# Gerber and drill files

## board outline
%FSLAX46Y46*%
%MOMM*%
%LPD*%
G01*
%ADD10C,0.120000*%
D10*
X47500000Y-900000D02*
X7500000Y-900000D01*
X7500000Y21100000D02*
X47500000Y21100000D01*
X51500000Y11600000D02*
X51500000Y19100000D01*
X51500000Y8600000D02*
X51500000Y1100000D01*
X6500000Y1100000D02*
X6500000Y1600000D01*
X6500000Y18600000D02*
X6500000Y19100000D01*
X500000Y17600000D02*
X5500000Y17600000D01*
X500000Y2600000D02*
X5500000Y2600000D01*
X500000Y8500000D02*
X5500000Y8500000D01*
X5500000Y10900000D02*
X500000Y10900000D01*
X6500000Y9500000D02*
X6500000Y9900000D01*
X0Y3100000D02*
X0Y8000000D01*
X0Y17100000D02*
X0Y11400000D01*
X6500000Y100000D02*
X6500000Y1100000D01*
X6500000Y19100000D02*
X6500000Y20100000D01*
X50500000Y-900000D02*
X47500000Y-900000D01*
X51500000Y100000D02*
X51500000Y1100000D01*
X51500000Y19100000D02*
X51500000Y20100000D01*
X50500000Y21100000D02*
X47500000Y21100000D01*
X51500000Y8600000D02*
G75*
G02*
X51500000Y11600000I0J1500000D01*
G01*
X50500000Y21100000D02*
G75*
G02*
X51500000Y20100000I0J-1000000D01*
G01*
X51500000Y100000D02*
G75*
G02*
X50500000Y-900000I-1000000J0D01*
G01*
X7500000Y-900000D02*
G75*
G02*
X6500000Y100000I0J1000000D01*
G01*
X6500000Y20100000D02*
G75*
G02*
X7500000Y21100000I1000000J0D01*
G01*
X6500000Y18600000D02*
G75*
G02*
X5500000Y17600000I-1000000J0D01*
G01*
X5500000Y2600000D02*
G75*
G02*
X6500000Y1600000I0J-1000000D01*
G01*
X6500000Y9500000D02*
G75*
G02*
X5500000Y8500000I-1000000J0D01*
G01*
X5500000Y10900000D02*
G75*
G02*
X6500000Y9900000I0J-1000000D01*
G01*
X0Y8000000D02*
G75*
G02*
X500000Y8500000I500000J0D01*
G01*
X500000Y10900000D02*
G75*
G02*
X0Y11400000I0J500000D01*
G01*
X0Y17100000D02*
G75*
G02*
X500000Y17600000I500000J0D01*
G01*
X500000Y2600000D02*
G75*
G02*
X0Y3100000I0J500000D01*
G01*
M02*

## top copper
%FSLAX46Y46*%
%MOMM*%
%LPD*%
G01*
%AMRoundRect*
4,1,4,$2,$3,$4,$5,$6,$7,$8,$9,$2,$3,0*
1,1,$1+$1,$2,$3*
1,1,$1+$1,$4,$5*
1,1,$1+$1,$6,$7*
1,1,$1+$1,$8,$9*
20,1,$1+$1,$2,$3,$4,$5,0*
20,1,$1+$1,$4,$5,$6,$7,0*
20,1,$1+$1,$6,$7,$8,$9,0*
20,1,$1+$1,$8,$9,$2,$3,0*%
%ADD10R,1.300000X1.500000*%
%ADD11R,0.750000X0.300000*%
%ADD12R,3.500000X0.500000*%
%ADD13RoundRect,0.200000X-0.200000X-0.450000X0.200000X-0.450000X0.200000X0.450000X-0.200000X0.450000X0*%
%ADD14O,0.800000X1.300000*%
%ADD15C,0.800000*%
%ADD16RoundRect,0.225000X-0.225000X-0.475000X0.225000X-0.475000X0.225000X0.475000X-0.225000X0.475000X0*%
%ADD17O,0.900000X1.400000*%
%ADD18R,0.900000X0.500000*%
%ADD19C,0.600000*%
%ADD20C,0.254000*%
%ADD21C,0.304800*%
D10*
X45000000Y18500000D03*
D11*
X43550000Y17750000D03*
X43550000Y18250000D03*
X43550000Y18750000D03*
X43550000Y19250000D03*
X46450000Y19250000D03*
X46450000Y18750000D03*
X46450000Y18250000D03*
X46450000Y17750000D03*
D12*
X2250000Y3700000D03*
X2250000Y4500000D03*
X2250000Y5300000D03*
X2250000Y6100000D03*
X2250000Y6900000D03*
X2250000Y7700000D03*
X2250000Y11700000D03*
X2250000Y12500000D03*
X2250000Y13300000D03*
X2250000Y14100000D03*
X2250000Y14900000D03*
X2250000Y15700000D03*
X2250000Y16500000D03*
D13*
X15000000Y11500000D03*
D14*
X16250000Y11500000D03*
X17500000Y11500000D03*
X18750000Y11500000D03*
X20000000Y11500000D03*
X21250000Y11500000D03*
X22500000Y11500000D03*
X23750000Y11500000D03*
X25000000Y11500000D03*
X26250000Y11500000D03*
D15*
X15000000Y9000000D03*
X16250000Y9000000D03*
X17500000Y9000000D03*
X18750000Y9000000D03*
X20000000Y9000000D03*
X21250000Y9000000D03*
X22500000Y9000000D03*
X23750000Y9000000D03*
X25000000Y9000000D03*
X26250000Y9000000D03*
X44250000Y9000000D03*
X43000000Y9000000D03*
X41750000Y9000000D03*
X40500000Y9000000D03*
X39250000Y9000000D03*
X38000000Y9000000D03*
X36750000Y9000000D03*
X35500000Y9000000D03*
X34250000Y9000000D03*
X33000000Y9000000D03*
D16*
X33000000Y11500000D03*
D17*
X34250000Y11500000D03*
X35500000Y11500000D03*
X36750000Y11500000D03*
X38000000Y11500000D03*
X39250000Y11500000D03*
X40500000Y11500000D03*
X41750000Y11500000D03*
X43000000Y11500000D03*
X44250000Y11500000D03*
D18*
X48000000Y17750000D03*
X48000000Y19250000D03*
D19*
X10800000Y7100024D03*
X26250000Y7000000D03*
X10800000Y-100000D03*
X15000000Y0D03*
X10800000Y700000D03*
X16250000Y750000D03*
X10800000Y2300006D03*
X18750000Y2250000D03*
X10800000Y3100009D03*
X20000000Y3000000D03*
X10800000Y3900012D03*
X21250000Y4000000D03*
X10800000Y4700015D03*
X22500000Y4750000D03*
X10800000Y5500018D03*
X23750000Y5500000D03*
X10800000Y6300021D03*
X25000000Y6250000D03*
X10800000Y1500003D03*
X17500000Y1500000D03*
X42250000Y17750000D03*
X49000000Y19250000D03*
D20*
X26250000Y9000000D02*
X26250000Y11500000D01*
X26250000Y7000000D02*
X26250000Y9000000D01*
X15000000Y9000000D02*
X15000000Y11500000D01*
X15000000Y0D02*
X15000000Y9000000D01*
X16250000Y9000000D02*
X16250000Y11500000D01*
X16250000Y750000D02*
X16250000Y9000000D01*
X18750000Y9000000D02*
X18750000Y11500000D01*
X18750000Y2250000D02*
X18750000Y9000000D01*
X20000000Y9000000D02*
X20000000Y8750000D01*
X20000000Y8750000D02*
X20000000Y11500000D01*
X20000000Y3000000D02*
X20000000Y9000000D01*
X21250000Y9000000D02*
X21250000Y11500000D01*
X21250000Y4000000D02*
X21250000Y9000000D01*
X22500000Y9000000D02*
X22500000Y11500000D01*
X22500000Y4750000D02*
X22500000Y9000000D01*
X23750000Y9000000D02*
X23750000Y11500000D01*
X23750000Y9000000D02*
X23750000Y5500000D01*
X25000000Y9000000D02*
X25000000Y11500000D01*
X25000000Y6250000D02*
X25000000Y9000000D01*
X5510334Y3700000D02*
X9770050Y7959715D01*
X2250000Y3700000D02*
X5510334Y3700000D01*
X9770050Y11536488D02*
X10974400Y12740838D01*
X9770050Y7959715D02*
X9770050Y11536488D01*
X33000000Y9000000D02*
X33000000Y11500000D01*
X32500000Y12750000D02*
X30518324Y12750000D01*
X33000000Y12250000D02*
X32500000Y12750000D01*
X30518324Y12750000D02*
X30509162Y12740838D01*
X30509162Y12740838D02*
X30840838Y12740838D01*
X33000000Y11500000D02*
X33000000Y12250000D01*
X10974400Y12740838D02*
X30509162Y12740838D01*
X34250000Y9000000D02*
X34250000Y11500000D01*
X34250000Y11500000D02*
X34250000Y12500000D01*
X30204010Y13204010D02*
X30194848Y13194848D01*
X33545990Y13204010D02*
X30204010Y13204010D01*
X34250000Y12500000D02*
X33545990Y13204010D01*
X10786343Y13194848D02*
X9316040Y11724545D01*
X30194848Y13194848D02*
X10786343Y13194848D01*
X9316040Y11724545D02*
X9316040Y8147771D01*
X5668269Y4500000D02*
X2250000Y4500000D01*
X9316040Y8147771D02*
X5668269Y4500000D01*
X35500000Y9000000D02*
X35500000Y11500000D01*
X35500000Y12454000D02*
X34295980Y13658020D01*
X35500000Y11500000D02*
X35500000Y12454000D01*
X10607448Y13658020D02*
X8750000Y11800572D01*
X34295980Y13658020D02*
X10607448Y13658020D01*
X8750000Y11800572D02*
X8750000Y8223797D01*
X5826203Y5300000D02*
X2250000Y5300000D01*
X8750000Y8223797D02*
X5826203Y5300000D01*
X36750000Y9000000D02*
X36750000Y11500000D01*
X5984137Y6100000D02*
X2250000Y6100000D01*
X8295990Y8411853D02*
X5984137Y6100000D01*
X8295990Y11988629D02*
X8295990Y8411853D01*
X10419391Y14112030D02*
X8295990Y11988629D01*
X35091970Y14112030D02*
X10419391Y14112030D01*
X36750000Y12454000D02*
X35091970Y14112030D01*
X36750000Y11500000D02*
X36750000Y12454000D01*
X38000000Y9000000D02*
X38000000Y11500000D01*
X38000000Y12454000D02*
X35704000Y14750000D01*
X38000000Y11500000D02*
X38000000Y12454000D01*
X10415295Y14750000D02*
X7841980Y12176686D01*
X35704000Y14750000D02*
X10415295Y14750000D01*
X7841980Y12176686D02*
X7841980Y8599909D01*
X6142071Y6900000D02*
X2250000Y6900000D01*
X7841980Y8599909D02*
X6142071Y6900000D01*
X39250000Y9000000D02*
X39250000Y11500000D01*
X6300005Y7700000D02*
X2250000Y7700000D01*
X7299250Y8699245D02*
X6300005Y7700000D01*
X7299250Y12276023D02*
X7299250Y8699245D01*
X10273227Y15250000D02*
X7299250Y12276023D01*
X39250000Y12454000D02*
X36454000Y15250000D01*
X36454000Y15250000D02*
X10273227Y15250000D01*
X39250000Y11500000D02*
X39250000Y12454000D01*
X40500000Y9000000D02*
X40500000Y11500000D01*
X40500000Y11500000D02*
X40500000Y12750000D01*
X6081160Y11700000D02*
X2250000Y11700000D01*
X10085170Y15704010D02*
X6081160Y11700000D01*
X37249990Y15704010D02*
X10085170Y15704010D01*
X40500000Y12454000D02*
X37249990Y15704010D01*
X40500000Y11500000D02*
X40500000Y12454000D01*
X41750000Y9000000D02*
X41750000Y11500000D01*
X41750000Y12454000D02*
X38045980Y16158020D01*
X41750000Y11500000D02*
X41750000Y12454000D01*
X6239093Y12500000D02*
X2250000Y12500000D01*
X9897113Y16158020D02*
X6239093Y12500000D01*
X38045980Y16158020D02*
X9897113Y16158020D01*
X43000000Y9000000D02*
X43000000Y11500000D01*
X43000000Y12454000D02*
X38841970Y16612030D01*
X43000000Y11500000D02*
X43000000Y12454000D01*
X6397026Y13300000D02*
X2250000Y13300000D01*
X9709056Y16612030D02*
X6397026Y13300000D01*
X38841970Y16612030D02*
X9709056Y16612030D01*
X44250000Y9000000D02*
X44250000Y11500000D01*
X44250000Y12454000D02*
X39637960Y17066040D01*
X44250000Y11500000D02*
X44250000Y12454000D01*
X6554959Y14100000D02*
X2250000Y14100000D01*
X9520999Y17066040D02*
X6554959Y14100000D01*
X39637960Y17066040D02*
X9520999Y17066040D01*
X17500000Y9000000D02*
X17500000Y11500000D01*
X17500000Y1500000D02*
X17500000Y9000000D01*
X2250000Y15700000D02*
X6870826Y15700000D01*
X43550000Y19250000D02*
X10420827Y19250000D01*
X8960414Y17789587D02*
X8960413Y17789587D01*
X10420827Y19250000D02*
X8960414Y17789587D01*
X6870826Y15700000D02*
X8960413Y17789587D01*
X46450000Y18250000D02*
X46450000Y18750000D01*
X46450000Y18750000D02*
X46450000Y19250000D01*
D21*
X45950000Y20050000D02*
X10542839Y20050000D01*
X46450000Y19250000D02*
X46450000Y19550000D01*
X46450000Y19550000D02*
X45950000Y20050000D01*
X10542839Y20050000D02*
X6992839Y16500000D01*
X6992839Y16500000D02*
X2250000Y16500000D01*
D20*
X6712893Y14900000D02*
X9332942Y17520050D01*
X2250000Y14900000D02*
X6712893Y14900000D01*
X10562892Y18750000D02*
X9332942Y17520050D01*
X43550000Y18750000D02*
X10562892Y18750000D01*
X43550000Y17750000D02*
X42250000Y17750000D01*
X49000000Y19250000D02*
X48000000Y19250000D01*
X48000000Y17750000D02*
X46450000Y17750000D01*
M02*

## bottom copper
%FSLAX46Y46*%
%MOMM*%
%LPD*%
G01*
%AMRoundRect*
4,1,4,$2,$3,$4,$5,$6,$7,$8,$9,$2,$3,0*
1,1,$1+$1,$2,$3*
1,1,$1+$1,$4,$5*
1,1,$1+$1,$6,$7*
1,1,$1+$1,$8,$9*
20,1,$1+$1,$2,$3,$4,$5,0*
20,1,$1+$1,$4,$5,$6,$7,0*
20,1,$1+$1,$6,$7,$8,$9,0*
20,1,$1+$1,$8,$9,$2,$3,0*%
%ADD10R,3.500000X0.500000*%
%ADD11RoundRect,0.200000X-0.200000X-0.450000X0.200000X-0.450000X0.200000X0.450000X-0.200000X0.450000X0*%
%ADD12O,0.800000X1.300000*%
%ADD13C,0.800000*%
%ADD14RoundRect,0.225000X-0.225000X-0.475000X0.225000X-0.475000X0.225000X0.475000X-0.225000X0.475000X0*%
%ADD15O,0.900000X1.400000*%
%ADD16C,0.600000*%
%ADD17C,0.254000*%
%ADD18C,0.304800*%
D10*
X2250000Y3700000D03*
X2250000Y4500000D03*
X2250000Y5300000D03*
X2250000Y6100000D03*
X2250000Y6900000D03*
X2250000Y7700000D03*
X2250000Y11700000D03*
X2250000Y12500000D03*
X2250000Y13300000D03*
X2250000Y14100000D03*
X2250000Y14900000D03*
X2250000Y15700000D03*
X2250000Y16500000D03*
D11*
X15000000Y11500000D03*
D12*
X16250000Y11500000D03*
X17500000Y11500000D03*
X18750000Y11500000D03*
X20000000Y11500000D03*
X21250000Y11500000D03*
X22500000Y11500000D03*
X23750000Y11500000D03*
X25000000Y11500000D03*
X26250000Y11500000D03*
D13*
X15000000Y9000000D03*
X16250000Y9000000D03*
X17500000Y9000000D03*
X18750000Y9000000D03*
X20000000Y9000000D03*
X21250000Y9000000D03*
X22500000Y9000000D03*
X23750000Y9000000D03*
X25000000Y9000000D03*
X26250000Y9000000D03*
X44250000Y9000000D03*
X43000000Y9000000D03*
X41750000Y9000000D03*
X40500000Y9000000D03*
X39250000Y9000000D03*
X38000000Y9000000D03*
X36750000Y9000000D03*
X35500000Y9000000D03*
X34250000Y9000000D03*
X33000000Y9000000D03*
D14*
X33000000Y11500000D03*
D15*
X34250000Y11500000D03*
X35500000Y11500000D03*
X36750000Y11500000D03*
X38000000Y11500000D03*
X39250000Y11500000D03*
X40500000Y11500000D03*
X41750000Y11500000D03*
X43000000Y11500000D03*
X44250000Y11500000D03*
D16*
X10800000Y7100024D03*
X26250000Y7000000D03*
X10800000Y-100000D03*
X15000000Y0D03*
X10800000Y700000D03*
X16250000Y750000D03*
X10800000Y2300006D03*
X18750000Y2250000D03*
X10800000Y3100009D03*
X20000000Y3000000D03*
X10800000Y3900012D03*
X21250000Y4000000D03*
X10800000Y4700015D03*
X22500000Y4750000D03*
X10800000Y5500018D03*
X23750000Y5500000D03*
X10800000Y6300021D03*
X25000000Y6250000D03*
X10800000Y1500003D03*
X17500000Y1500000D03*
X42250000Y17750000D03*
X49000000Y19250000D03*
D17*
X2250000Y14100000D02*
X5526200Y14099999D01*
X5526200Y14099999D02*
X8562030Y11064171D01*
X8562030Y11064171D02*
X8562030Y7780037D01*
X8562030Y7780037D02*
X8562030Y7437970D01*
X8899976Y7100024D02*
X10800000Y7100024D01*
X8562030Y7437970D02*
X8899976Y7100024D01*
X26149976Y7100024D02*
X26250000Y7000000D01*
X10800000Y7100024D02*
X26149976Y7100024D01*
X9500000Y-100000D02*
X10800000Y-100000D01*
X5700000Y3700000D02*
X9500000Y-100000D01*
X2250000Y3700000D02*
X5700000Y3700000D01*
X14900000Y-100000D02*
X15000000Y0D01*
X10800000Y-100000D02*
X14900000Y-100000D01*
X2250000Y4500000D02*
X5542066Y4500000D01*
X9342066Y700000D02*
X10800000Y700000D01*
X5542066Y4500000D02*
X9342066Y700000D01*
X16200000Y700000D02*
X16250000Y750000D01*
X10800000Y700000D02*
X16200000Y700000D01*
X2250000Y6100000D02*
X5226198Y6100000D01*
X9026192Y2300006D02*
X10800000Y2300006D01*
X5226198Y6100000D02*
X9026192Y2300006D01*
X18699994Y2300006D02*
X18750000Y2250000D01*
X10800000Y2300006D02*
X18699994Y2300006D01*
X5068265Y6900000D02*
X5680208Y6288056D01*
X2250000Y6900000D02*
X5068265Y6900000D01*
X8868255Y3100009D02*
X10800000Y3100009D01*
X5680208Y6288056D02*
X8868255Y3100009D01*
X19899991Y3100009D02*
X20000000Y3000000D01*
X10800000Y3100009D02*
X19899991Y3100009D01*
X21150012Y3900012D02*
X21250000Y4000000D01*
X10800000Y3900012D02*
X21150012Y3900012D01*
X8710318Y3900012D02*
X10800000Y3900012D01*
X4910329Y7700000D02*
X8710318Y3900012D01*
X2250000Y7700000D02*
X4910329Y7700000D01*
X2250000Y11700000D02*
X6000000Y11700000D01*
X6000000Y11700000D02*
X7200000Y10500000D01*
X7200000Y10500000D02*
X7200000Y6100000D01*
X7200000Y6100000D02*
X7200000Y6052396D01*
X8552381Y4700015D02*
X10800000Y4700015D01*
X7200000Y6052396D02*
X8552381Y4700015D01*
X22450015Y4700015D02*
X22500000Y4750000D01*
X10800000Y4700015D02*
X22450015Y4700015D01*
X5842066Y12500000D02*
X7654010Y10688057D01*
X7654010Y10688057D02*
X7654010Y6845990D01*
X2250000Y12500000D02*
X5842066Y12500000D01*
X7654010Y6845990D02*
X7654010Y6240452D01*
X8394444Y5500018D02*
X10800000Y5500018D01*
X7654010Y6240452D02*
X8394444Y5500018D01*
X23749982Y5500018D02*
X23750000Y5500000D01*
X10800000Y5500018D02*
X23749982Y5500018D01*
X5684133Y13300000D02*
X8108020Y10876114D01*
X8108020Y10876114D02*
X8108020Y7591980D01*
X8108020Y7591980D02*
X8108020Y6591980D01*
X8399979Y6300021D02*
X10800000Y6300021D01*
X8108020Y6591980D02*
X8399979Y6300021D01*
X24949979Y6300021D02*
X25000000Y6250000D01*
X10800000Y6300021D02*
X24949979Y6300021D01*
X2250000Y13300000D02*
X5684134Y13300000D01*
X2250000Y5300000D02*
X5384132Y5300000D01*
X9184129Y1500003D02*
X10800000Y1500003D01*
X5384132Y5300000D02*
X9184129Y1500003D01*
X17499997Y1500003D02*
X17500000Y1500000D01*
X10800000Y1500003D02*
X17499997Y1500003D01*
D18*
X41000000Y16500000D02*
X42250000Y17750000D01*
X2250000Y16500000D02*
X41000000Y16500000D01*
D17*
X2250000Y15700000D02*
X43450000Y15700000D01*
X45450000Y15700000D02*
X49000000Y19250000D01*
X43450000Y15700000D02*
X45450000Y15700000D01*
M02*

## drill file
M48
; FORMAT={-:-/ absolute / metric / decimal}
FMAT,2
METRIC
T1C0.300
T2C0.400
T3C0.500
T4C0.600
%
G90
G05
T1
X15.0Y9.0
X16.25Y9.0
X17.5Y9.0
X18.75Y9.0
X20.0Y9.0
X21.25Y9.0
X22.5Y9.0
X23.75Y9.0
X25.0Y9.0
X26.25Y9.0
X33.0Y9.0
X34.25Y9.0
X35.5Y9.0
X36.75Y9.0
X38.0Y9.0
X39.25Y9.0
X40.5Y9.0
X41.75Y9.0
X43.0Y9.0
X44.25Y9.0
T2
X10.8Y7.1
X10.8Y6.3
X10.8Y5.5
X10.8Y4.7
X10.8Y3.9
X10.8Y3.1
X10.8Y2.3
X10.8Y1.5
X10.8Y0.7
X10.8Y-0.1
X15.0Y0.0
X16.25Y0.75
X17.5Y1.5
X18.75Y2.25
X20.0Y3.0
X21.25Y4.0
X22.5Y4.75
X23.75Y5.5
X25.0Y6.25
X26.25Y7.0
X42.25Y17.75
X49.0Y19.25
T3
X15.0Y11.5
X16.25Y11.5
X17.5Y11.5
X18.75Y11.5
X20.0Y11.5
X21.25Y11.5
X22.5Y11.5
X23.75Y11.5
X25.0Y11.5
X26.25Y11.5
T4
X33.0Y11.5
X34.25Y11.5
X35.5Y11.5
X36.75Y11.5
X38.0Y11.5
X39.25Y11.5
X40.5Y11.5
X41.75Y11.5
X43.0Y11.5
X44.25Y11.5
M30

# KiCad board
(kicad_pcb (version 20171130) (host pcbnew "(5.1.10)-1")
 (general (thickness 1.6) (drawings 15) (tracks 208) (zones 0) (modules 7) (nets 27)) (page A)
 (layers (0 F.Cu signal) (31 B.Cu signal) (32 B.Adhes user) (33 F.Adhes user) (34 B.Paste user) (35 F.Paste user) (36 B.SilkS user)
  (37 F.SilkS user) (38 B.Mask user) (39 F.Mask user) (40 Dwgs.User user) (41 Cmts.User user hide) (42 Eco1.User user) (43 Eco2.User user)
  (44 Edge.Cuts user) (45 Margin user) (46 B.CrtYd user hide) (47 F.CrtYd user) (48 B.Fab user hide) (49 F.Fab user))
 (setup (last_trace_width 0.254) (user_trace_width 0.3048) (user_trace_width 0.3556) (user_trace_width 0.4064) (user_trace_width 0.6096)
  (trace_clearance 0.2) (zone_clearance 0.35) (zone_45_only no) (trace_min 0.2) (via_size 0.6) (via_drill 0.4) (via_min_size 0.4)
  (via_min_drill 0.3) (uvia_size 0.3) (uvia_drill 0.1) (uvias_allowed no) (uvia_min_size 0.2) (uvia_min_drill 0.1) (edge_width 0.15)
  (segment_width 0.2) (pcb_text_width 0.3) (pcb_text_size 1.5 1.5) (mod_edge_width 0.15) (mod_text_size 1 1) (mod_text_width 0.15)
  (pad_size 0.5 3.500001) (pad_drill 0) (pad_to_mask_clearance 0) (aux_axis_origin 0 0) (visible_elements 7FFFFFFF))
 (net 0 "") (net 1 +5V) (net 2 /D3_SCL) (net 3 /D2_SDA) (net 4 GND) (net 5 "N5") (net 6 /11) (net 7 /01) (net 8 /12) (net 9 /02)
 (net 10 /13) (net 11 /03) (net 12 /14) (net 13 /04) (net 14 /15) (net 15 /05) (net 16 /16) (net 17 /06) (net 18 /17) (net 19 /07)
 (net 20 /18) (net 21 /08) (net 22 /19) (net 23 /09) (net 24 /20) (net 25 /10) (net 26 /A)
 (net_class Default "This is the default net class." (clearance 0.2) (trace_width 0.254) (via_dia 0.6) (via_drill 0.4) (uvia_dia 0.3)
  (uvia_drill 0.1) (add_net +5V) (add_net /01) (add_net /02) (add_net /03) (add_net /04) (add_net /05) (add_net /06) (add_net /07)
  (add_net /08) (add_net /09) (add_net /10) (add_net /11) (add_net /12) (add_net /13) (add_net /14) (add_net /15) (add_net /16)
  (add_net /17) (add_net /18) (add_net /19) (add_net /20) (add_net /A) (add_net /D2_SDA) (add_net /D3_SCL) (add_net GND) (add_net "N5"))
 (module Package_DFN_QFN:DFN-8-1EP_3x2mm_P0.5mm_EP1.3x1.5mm (layer F.Cu) (at 45 -18.5 180)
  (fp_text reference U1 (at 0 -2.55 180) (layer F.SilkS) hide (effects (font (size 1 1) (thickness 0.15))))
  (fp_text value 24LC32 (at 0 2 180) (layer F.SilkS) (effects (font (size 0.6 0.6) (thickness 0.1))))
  (pad "" smd rect (at 0.325 0.375 180) (size 0.5 0.6) (layers F.Paste))
  (pad "" smd rect (at 0.325 -0.375 180) (size 0.5 0.6) (layers F.Paste))
  (pad "" smd rect (at -0.325 0.375 180) (size 0.5 0.6) (layers F.Paste))
  (pad "" smd rect (at -0.325 -0.375 180) (size 0.5 0.6) (layers F.Paste))
  (pad 9 smd rect (at 0 0 180) (size 1.3 1.5) (layers F.Cu F.Mask))
  (pad 8 smd rect (at 1.45 -0.75 180) (size 0.75 0.3) (layers F.Cu F.Paste F.Mask) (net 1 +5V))
  (pad 7 smd rect (at 1.45 -0.25 180) (size 0.75 0.3) (layers F.Cu F.Paste F.Mask))
  (pad 6 smd rect (at 1.45 0.25 180) (size 0.75 0.3) (layers F.Cu F.Paste F.Mask) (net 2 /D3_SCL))
  (pad 5 smd rect (at 1.45 0.75 180) (size 0.75 0.3) (layers F.Cu F.Paste F.Mask) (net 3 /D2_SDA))
  (pad 4 smd rect (at -1.45 0.75 180) (size 0.75 0.3) (layers F.Cu F.Paste F.Mask) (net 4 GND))
  (pad 3 smd rect (at -1.45 0.25 180) (size 0.75 0.3) (layers F.Cu F.Paste F.Mask) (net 4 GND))
  (pad 2 smd rect (at -1.45 -0.25 180) (size 0.75 0.3) (layers F.Cu F.Paste F.Mask) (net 4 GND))
  (pad 1 smd rect (at -1.45 -0.75 180) (size 0.75 0.3) (layers F.Cu F.Paste F.Mask) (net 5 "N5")))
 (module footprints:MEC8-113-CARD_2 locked (layer F.Cu) (at 0 -0.1 90)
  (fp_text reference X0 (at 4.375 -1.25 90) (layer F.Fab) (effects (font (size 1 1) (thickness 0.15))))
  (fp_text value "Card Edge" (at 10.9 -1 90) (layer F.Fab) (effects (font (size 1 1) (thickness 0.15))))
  (fp_line (start -1 47.5) (end -1 7.5) (layer Edge.Cuts) (width 0.12))
  (fp_line (start 21 7.5) (end 21 47.5) (layer Edge.Cuts) (width 0.12))
  (fp_line (start 11.5 51.5) (end 19 51.5) (layer Edge.Cuts) (width 0.12))
  (fp_line (start 8.5 51.5) (end 1 51.5) (layer Edge.Cuts) (width 0.12))
  (fp_line (start 1 6.5) (end 1.5 6.5) (layer Edge.Cuts) (width 0.12))
  (fp_line (start 18.5 6.5) (end 19 6.5) (layer Edge.Cuts) (width 0.12))
  (fp_line (start 17.5 0.5) (end 17.5 5.5) (layer Edge.Cuts) (width 0.12))
  (fp_line (start 2.5 0.5) (end 2.5 5.5) (layer Edge.Cuts) (width 0.12))
  (fp_line (start 8.4 0.5) (end 8.4 5.5) (layer Edge.Cuts) (width 0.12))
  (fp_line (start 10.8 5.5) (end 10.8 0.5) (layer Edge.Cuts) (width 0.12))
  (fp_line (start 9.4 6.5) (end 9.8 6.5) (layer Edge.Cuts) (width 0.12))
  (fp_line (start 3 0) (end 7.9 0) (layer Edge.Cuts) (width 0.12))
  (fp_line (start 17 0) (end 11.3 0) (layer Edge.Cuts) (width 0.12))
  (fp_line (start 0 6.5) (end 1 6.5) (layer Edge.Cuts) (width 0.12))
  (fp_line (start 19 6.5) (end 20 6.5) (layer Edge.Cuts) (width 0.12))
  (fp_line (start -1 50.5) (end -1 47.5) (layer Edge.Cuts) (width 0.12))
  (fp_line (start 0 51.5) (end 1 51.5) (layer Edge.Cuts) (width 0.12))
  (fp_line (start 19 51.5) (end 20 51.5) (layer Edge.Cuts) (width 0.12))
  (fp_line (start 21 50.5) (end 21 47.5) (layer Edge.Cuts) (width 0.12))
  (fp_arc (start 10 51.5) (end 11.5 51.5) (angle -180) (layer Edge.Cuts) (width 0.12))
  (fp_arc (start 20 50.5) (end 20 51.5) (angle -90) (layer Edge.Cuts) (width 0.12))
  (fp_arc (start 0 50.5) (end -1 50.5) (angle -90) (layer Edge.Cuts) (width 0.12))
  (fp_arc (start 0 7.5) (end 0 6.5) (angle -90) (layer Edge.Cuts) (width 0.12))
  (fp_arc (start 20 7.5) (end 21 7.5) (angle -90) (layer Edge.Cuts) (width 0.12))
  (fp_arc (start 18.5 5.5) (end 17.5 5.5) (angle -90) (layer Edge.Cuts) (width 0.12))
  (fp_arc (start 1.5 5.5) (end 1.5 6.5) (angle -90) (layer Edge.Cuts) (width 0.12))
  (fp_arc (start 9.4 5.5) (end 8.4 5.5) (angle -90) (layer Edge.Cuts) (width 0.12))
  (fp_arc (start 9.8 5.5) (end 9.8 6.5) (angle -90) (layer Edge.Cuts) (width 0.12))
  (fp_arc (start 7.9 0.5) (end 8.4 0.5) (angle -90) (layer Edge.Cuts) (width 0.12))
  (fp_arc (start 11.3 0.5) (end 11.3 0) (angle -90) (layer Edge.Cuts) (width 0.12))
  (fp_arc (start 17 0.5) (end 17.5 0.5) (angle -90) (layer Edge.Cuts) (width 0.12))
  (fp_arc (start 3 0.5) (end 3 0) (angle -90) (layer Edge.Cuts) (width 0.12))
  (pad 14 smd rect (at 3.6 2.25 90) (size 0.5 3.5) (layers F.Cu F.Paste F.Mask) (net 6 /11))
  (pad 1 smd rect (at 3.6 2.25 90) (size 0.5 3.5) (layers B.Cu B.Paste B.Mask) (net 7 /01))
  (pad 15 smd rect (at 4.4 2.25 90) (size 0.5 3.5) (layers F.Cu F.Paste F.Mask) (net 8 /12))
  (pad 2 smd rect (at 4.4 2.25 90) (size 0.5 3.5) (layers B.Cu B.Paste B.Mask) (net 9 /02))
  (pad 16 smd rect (at 5.2 2.25 90) (size 0.5 3.5) (layers F.Cu F.Paste F.Mask) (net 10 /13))
  (pad 3 smd rect (at 5.2 2.25 90) (size 0.5 3.5) (layers B.Cu B.Paste B.Mask) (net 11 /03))
  (pad 17 smd rect (at 6 2.25 90) (size 0.5 3.5) (layers F.Cu F.Paste F.Mask) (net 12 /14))
  (pad 4 smd rect (at 6 2.25 90) (size 0.5 3.5) (layers B.Cu B.Paste B.Mask) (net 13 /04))
  (pad 18 smd rect (at 6.8 2.25 90) (size 0.5 3.5) (layers F.Cu F.Paste F.Mask) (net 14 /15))
  (pad 5 smd rect (at 6.8 2.25 90) (size 0.5 3.5) (layers B.Cu B.Paste B.Mask) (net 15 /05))
  (pad 19 smd rect (at 7.6 2.25 90) (size 0.5 3.5) (layers F.Cu F.Paste F.Mask) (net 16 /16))
  (pad 6 smd rect (at 7.6 2.25 90) (size 0.5 3.5) (layers B.Cu B.Paste B.Mask) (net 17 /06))
  (pad 20 smd rect (at 11.6 2.25 90) (size 0.5 3.5) (layers F.Cu F.Paste F.Mask) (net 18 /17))
  (pad 7 smd rect (at 11.6 2.25 90) (size 0.5 3.5) (layers B.Cu B.Paste B.Mask) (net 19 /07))
  (pad 21 smd rect (at 12.4 2.25 90) (size 0.5 3.5) (layers F.Cu F.Paste F.Mask) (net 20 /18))
  (pad 8 smd rect (at 12.4 2.25 90) (size 0.5 3.5) (layers B.Cu B.Paste B.Mask) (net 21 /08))
  (pad 22 smd rect (at 13.2 2.25 90) (size 0.5 3.5) (layers F.Cu F.Paste F.Mask) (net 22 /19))
  (pad 9 smd rect (at 13.2 2.25 90) (size 0.5 3.5) (layers B.Cu B.Paste B.Mask) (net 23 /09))
  (pad 23 smd rect (at 14 2.25 90) (size 0.5 3.5) (layers F.Cu F.Paste F.Mask) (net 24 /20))
  (pad 10 smd rect (at 14 2.25 90) (size 0.5 3.5) (layers B.Cu B.Paste B.Mask) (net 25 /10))
  (pad 24 smd rect (at 14.8 2.25 90) (size 0.5 3.5) (layers F.Cu F.Paste F.Mask) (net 2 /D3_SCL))
  (pad 11 smd rect (at 14.8 2.25 90) (size 0.5 3.5) (layers B.Cu B.Paste B.Mask))
  (pad 25 smd rect (at 15.6 2.25 90) (size 0.5 3.5) (layers F.Cu F.Paste F.Mask) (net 3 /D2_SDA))
  (pad 12 smd rect (at 15.6 2.25 90) (size 0.5 3.5) (layers B.Cu B.Paste B.Mask) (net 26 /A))
  (pad 26 smd rect (at 16.4 2.25 90) (size 0.5 3.5) (layers F.Cu F.Paste F.Mask) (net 4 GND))
  (pad 13 smd rect (at 16.4 2.25 90) (size 0.5 3.5) (layers B.Cu B.Paste B.Mask) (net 1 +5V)))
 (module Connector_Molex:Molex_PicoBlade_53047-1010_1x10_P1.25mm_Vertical (layer F.Cu) (at 15 -11.5)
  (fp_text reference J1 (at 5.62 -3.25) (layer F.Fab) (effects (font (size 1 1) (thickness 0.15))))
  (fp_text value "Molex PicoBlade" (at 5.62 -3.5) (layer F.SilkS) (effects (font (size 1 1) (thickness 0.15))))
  (pad 1 thru_hole roundrect (at 0 0) (size 0.8 1.3) (drill 0.5) (layers *.Cu *.Mask) (roundrect_rratio 0.25) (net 7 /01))
  (pad 2 thru_hole oval (at 1.25 0) (size 0.8 1.3) (drill 0.5) (layers *.Cu *.Mask) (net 9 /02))
  (pad 3 thru_hole oval (at 2.5 0) (size 0.8 1.3) (drill 0.5) (layers *.Cu *.Mask) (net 11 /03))
  (pad 4 thru_hole oval (at 3.75 0) (size 0.8 1.3) (drill 0.5) (layers *.Cu *.Mask) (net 13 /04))
  (pad 5 thru_hole oval (at 5 0) (size 0.8 1.3) (drill 0.5) (layers *.Cu *.Mask) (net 15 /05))
  (pad 6 thru_hole oval (at 6.25 0) (size 0.8 1.3) (drill 0.5) (layers *.Cu *.Mask) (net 17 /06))
  (pad 7 thru_hole oval (at 7.5 0) (size 0.8 1.3) (drill 0.5) (layers *.Cu *.Mask) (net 19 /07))
  (pad 8 thru_hole oval (at 8.75 0) (size 0.8 1.3) (drill 0.5) (layers *.Cu *.Mask) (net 21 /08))
  (pad 9 thru_hole oval (at 10 0) (size 0.8 1.3) (drill 0.5) (layers *.Cu *.Mask) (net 23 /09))
  (pad 10 thru_hole oval (at 11.25 0) (size 0.8 1.3) (drill 0.5) (layers *.Cu *.Mask) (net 25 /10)))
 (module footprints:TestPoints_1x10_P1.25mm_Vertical (layer F.Cu) (at 15 -9)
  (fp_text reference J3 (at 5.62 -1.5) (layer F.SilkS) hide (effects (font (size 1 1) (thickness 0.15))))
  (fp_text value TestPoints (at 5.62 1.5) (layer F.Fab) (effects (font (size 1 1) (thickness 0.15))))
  (pad 1 thru_hole circle (at 0 0) (size 0.8 0.8) (drill 0.3) (layers *.Cu *.Mask) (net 7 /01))
  (pad 2 thru_hole circle (at 1.25 0) (size 0.8 0.8) (drill 0.3) (layers *.Cu *.Mask) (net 9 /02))
  (pad 3 thru_hole circle (at 2.5 0) (size 0.8 0.8) (drill 0.3) (layers *.Cu *.Mask) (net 11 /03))
  (pad 4 thru_hole circle (at 3.75 0) (size 0.8 0.8) (drill 0.3) (layers *.Cu *.Mask) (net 13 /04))
  (pad 5 thru_hole circle (at 5 0) (size 0.8 0.8) (drill 0.3) (layers *.Cu *.Mask) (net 15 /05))
  (pad 6 thru_hole circle (at 6.25 0) (size 0.8 0.8) (drill 0.3) (layers *.Cu *.Mask) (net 17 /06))
  (pad 7 thru_hole circle (at 7.5 0) (size 0.8 0.8) (drill 0.3) (layers *.Cu *.Mask) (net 19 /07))
  (pad 8 thru_hole circle (at 8.75 0) (size 0.8 0.8) (drill 0.3) (layers *.Cu *.Mask) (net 21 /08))
  (pad 9 thru_hole circle (at 10 0) (size 0.8 0.8) (drill 0.3) (layers *.Cu *.Mask) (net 23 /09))
  (pad 10 thru_hole circle (at 11.25 0) (size 0.8 0.8) (drill 0.3) (layers *.Cu *.Mask) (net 25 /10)))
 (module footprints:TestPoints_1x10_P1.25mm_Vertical (layer F.Cu) (at 33 -9)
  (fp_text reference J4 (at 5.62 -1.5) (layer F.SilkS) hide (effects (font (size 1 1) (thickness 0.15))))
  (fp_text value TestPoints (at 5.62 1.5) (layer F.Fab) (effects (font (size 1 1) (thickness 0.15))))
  (pad 10 thru_hole circle (at 11.25 0) (size 0.8 0.8) (drill 0.3) (layers *.Cu *.Mask) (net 24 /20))
  (pad 9 thru_hole circle (at 10 0) (size 0.8 0.8) (drill 0.3) (layers *.Cu *.Mask) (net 22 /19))
  (pad 8 thru_hole circle (at 8.75 0) (size 0.8 0.8) (drill 0.3) (layers *.Cu *.Mask) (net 20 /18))
  (pad 7 thru_hole circle (at 7.5 0) (size 0.8 0.8) (drill 0.3) (layers *.Cu *.Mask) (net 18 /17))
  (pad 6 thru_hole circle (at 6.25 0) (size 0.8 0.8) (drill 0.3) (layers *.Cu *.Mask) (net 16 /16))
  (pad 5 thru_hole circle (at 5 0) (size 0.8 0.8) (drill 0.3) (layers *.Cu *.Mask) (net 14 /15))
  (pad 4 thru_hole circle (at 3.75 0) (size 0.8 0.8) (drill 0.3) (layers *.Cu *.Mask) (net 12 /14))
  (pad 3 thru_hole circle (at 2.5 0) (size 0.8 0.8) (drill 0.3) (layers *.Cu *.Mask) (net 10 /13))
  (pad 2 thru_hole circle (at 1.25 0) (size 0.8 0.8) (drill 0.3) (layers *.Cu *.Mask) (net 8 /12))
  (pad 1 thru_hole circle (at 0 0) (size 0.8 0.8) (drill 0.3) (layers *.Cu *.Mask) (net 6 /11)))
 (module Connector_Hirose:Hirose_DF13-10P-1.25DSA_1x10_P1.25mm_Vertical (layer F.Cu) (at 33 -11.5)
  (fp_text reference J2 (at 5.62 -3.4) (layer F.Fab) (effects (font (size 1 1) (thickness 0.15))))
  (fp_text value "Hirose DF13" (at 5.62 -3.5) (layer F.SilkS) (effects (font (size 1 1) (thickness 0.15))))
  (pad 1 thru_hole roundrect (at 0 0) (size 0.9 1.4) (drill 0.6) (layers *.Cu *.Mask) (roundrect_rratio 0.25) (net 6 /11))
  (pad 2 thru_hole oval (at 1.25 0) (size 0.9 1.4) (drill 0.6) (layers *.Cu *.Mask) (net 8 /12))
  (pad 3 thru_hole oval (at 2.5 0) (size 0.9 1.4) (drill 0.6) (layers *.Cu *.Mask) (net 10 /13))
  (pad 4 thru_hole oval (at 3.75 0) (size 0.9 1.4) (drill 0.6) (layers *.Cu *.Mask) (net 12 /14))
  (pad 5 thru_hole oval (at 5 0) (size 0.9 1.4) (drill 0.6) (layers *.Cu *.Mask) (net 14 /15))
  (pad 6 thru_hole oval (at 6.25 0) (size 0.9 1.4) (drill 0.6) (layers *.Cu *.Mask) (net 16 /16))
  (pad 7 thru_hole oval (at 7.5 0) (size 0.9 1.4) (drill 0.6) (layers *.Cu *.Mask) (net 18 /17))
  (pad 8 thru_hole oval (at 8.75 0) (size 0.9 1.4) (drill 0.6) (layers *.Cu *.Mask) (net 20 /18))
  (pad 9 thru_hole oval (at 10 0) (size 0.9 1.4) (drill 0.6) (layers *.Cu *.Mask) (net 22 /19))
  (pad 10 thru_hole oval (at 11.25 0) (size 0.9 1.4) (drill 0.6) (layers *.Cu *.Mask) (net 24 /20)))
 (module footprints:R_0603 (layer F.Cu) (at 48 -18.5 90)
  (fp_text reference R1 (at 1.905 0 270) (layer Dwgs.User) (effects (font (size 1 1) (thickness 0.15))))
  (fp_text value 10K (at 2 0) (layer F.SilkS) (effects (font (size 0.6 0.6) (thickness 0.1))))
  (pad 1 smd rect (at -0.75 0 90) (size 0.5 0.9) (layers F.Cu F.Paste F.Mask) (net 5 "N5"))
  (pad 2 smd rect (at 0.75 0 90) (size 0.5 0.9) (layers F.Cu F.Paste F.Mask) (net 26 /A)))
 (segment (start 2.25 -14.1) (end 5.5262 -14.099999) (width 0.254) (layer B.Cu) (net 25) (status 10))
 (segment (start 5.5262 -14.099999) (end 8.56203 -11.064171) (width 0.254) (layer B.Cu) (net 25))
 (segment (start 8.56203 -11.064171) (end 8.56203 -7.780037) (width 0.254) (layer B.Cu) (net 25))
 (segment (start 8.56203 -7.780037) (end 8.56203 -7.43797) (width 0.254) (layer B.Cu) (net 25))
 (via (at 10.8 -7.100024) (size 0.6) (drill 0.4) (layers F.Cu B.Cu) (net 25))
 (segment (start 8.899976 -7.100024) (end 10.8 -7.100024) (width 0.254) (layer B.Cu) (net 25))
 (segment (start 8.56203 -7.43797) (end 8.899976 -7.100024) (width 0.254) (layer B.Cu) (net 25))
 (segment (start 26.25 -9) (end 26.25 -11.5) (width 0.254) (layer F.Cu) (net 25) (status 30))
 (via (at 26.25 -7) (size 0.6) (drill 0.4) (layers F.Cu B.Cu) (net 25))
 (segment (start 26.149976 -7.100024) (end 26.25 -7) (width 0.254) (layer B.Cu) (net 25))
 (segment (start 10.8 -7.100024) (end 26.149976 -7.100024) (width 0.254) (layer B.Cu) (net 25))
 (segment (start 26.25 -7) (end 26.25 -9) (width 0.254) (layer F.Cu) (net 25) (status 20))
 (via (at 10.8 0.1) (size 0.6) (drill 0.4) (layers F.Cu B.Cu) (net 7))
 (segment (start 9.5 0.1) (end 10.8 0.1) (width 0.254) (layer B.Cu) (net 7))
 (segment (start 5.7 -3.7) (end 9.5 0.1) (width 0.254) (layer B.Cu) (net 7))
 (segment (start 2.25 -3.7) (end 5.7 -3.7) (width 0.254) (layer B.Cu) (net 7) (status 10))
 (segment (start 15 -9) (end 15 -11.5) (width 0.254) (layer F.Cu) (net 7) (status 30))
 (via (at 15 0) (size 0.6) (drill 0.4) (layers F.Cu B.Cu) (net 7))
 (segment (start 14.9 0.1) (end 15 0) (width 0.254) (layer B.Cu) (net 7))
 (segment (start 10.8 0.1) (end 14.9 0.1) (width 0.254) (layer B.Cu) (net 7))
 (segment (start 15 0) (end 15 -9) (width 0.254) (layer F.Cu) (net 7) (status 20))
 (segment (start 2.25 -4.5) (end 5.542066 -4.5) (width 0.254) (layer B.Cu) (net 9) (status 10))
 (via (at 10.8 -0.7) (size 0.6) (drill 0.4) (layers F.Cu B.Cu) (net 9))
 (segment (start 9.342066 -0.7) (end 10.8 -0.7) (width 0.254) (layer B.Cu) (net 9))
 (segment (start 5.542066 -4.5) (end 9.342066 -0.7) (width 0.254) (layer B.Cu) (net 9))
 (segment (start 16.25 -9) (end 16.25 -11.5) (width 0.254) (layer F.Cu) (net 9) (status 30))
 (via (at 16.25 -0.75) (size 0.6) (drill 0.4) (layers F.Cu B.Cu) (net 9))
 (segment (start 16.2 -0.7) (end 16.25 -0.75) (width 0.254) (layer B.Cu) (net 9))
 (segment (start 10.8 -0.7) (end 16.2 -0.7) (width 0.254) (layer B.Cu) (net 9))
 (segment (start 16.25 -0.75) (end 16.25 -9) (width 0.254) (layer F.Cu) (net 9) (status 20))
 (segment (start 2.25 -6.1) (end 5.226198 -6.1) (width 0.254) (layer B.Cu) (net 13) (status 10))
 (via (at 10.8 -2.300006) (size 0.6) (drill 0.4) (layers F.Cu B.Cu) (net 13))
 (segment (start 9.026192 -2.300006) (end 10.8 -2.300006) (width 0.254) (layer B.Cu) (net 13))
 (segment (start 5.226198 -6.1) (end 9.026192 -2.300006) (width 0.254) (layer B.Cu) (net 13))
 (segment (start 18.75 -9) (end 18.75 -11.5) (width 0.254) (layer F.Cu) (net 13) (status 30))
 (via (at 18.75 -2.25) (size 0.6) (drill 0.4) (layers F.Cu B.Cu) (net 13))
 (segment (start 18.699994 -2.300006) (end 18.75 -2.25) (width 0.254) (layer B.Cu) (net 13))
 (segment (start 10.8 -2.300006) (end 18.699994 -2.300006) (width 0.254) (layer B.Cu) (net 13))
 (segment (start 18.75 -2.25) (end 18.75 -9) (width 0.254) (layer F.Cu) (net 13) (status 20))
 (segment (start 5.068265 -6.9) (end 5.680208 -6.288056) (width 0.254) (layer B.Cu) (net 15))
 (segment (start 2.25 -6.9) (end 5.068265 -6.9) (width 0.254) (layer B.Cu) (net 15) (status 10))
 (via (at 10.8 -3.100009) (size 0.6) (drill 0.4) (layers F.Cu B.Cu) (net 15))
 (segment (start 8.868255 -3.100009) (end 10.8 -3.100009) (width 0.254) (layer B.Cu) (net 15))
 (segment (start 5.680208 -6.288056) (end 8.868255 -3.100009) (width 0.254) (layer B.Cu) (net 15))
 (segment (start 20 -9) (end 20 -8.75) (width 0.254) (layer F.Cu) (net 15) (status 30))
 (segment (start 20 -8.75) (end 20 -11.5) (width 0.254) (layer F.Cu) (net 15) (status 30))
 (via (at 20 -3) (size 0.6) (drill 0.4) (layers F.Cu B.Cu) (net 15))
 (segment (start 19.899991 -3.100009) (end 20 -3) (width 0.254) (layer B.Cu) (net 15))
 (segment (start 10.8 -3.100009) (end 19.899991 -3.100009) (width 0.254) (layer B.Cu) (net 15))
 (segment (start 20 -3) (end 20 -9) (width 0.254) (layer F.Cu) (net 15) (status 20))
 (via (at 10.8 -3.900012) (size 0.6) (drill 0.4) (layers F.Cu B.Cu) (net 17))
 (segment (start 21.25 -9) (end 21.25 -11.5) (width 0.254) (layer F.Cu) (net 17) (status 30))
 (via (at 21.25 -4) (size 0.6) (drill 0.4) (layers F.Cu B.Cu) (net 17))
 (segment (start 21.150012 -3.900012) (end 21.25 -4) (width 0.254) (layer B.Cu) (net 17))
 (segment (start 10.8 -3.900012) (end 21.150012 -3.900012) (width 0.254) (layer B.Cu) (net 17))
 (segment (start 21.25 -4) (end 21.25 -9) (width 0.254) (layer F.Cu) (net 17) (status 20))
 (segment (start 8.710318 -3.900012) (end 10.8 -3.900012) (width 0.254) (layer B.Cu) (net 17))
 (segment (start 4.910329 -7.7) (end 8.710318 -3.900012) (width 0.254) (layer B.Cu) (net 17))
 (segment (start 2.25 -7.7) (end 4.910329 -7.7) (width 0.254) (layer B.Cu) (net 17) (status 10))
 (segment (start 2.25 -11.7) (end 6 -11.7) (width 0.254) (layer B.Cu) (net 19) (status 10))
 (segment (start 6 -11.7) (end 7.2 -10.5) (width 0.254) (layer B.Cu) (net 19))
 (segment (start 7.2 -10.5) (end 7.2 -6.1) (width 0.254) (layer B.Cu) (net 19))
 (segment (start 7.2 -6.1) (end 7.2 -6.052396) (width 0.254) (layer B.Cu) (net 19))
 (via (at 10.8 -4.700015) (size 0.6) (drill 0.4) (layers F.Cu B.Cu) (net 19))
 (segment (start 8.552381 -4.700015) (end 10.8 -4.700015) (width 0.254) (layer B.Cu) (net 19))
 (segment (start 7.2 -6.052396) (end 8.552381 -4.700015) (width 0.254) (layer B.Cu) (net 19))
 (segment (start 22.5 -9) (end 22.5 -11.5) (width 0.254) (layer F.Cu) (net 19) (status 30))
 (segment (start 22.450015 -4.700015) (end 22.5 -4.75) (width 0.254) (layer B.Cu) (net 19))
 (via (at 22.5 -4.75) (size 0.6) (drill 0.4) (layers F.Cu B.Cu) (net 19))
 (segment (start 10.8 -4.700015) (end 22.450015 -4.700015) (width 0.254) (layer B.Cu) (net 19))
 (segment (start 22.5 -4.75) (end 22.5 -9) (width 0.254) (layer F.Cu) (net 19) (status 20))
 (segment (start 5.842066 -12.5) (end 7.65401 -10.688057) (width 0.254) (layer B.Cu) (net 21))
 (segment (start 7.65401 -10.688057) (end 7.65401 -6.84599) (width 0.254) (layer B.Cu) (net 21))
 (segment (start 2.25 -12.5) (end 5.842066 -12.5) (width 0.254) (layer B.Cu) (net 21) (status 10))
 (segment (start 7.65401 -6.84599) (end 7.65401 -6.240452) (width 0.254) (layer B.Cu) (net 21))
 (segment (start 8.394444 -5.500018) (end 10.8 -5.500018) (width 0.254) (layer B.Cu) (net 21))
 (via (at 10.8 -5.500018) (size 0.6) (drill 0.4) (layers F.Cu B.Cu) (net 21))
 (segment (start 7.65401 -6.240452) (end 8.394444 -5.500018) (width 0.254) (layer B.Cu) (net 21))
 (segment (start 23.75 -9) (end 23.75 -11.5) (width 0.254) (layer F.Cu) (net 21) (status 30))
 (via (at 23.75 -5.5) (size 0.6) (drill 0.4) (layers F.Cu B.Cu) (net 21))
 (segment (start 23.749982 -5.500018) (end 23.75 -5.5) (width 0.254) (layer B.Cu) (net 21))
 (segment (start 10.8 -5.500018) (end 23.749982 -5.500018) (width 0.254) (layer B.Cu) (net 21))
 (segment (start 23.75 -9) (end 23.75 -5.5) (width 0.254) (layer F.Cu) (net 21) (status 10))
 (segment (start 5.684133 -13.3) (end 8.10802 -10.876114) (width 0.254) (layer B.Cu) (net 23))
 (segment (start 8.10802 -10.876114) (end 8.10802 -7.59198) (width 0.254) (layer B.Cu) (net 23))
 (segment (start 8.10802 -7.59198) (end 8.10802 -6.59198) (width 0.254) (layer B.Cu) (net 23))
 (via (at 10.8 -6.300021) (size 0.6) (drill 0.4) (layers F.Cu B.Cu) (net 23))
 (segment (start 8.399979 -6.300021) (end 10.8 -6.300021) (width 0.254) (layer B.Cu) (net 23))
 (segment (start 8.10802 -6.59198) (end 8.399979 -6.300021) (width 0.254) (layer B.Cu) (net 23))
 (segment (start 25 -9) (end 25 -11.5) (width 0.254) (layer F.Cu) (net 23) (status 30))
 (via (at 25 -6.25) (size 0.6) (drill 0.4) (layers F.Cu B.Cu) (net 23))
 (segment (start 24.949979 -6.300021) (end 25 -6.25) (width 0.254) (layer B.Cu) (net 23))
 (segment (start 10.8 -6.300021) (end 24.949979 -6.300021) (width 0.254) (layer B.Cu) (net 23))
 (segment (start 25 -6.25) (end 25 -9) (width 0.254) (layer F.Cu) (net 23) (status 20))
 (segment (start 2.25 -13.3) (end 5.684134 -13.3) (width 0.254) (layer B.Cu) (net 23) (status 10))
 (segment (start 5.510334 -3.7) (end 9.77005 -7.959715) (width 0.254) (layer F.Cu) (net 6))
 (segment (start 2.25 -3.7) (end 5.510334 -3.7) (width 0.254) (layer F.Cu) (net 6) (status 10))
 (segment (start 9.77005 -11.536488) (end 10.9744 -12.740838) (width 0.254) (layer F.Cu) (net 6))
 (segment (start 9.77005 -7.959715) (end 9.77005 -11.536488) (width 0.254) (layer F.Cu) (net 6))
 (segment (start 33 -9) (end 33 -11.5) (width 0.254) (layer F.Cu) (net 6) (status 30))
 (segment (start 32.5 -12.75) (end 30.518324 -12.75) (width 0.254) (layer F.Cu) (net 6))
 (segment (start 33 -12.25) (end 32.5 -12.75) (width 0.254) (layer F.Cu) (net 6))
 (segment (start 30.518324 -12.75) (end 30.509162 -12.740838) (width 0.254) (layer F.Cu) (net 6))
 (segment (start 30.509162 -12.740838) (end 30.840838 -12.740838) (width 0.254) (layer F.Cu) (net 6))
 (segment (start 33 -11.5) (end 33 -12.25) (width 0.254) (layer F.Cu) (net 6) (status 10))
 (segment (start 10.9744 -12.740838) (end 30.509162 -12.740838) (width 0.254) (layer F.Cu) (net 6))
 (segment (start 34.25 -9) (end 34.25 -11.5) (width 0.254) (layer F.Cu) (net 8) (status 30))
 (segment (start 34.25 -11.5) (end 34.25 -12.5) (width 0.254) (layer F.Cu) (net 8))
 (segment (start 30.20401 -13.20401) (end 30.194848 -13.194848) (width 0.254) (layer F.Cu) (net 8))
 (segment (start 33.54599 -13.20401) (end 30.20401 -13.20401) (width 0.254) (layer F.Cu) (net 8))
 (segment (start 34.25 -12.5) (end 33.54599 -13.20401) (width 0.254) (layer F.Cu) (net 8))
 (segment (start 10.786343 -13.194848) (end 9.31604 -11.724545) (width 0.254) (layer F.Cu) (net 8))
 (segment (start 30.194848 -13.194848) (end 10.786343 -13.194848) (width 0.254) (layer F.Cu) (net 8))
 (segment (start 9.31604 -11.724545) (end 9.31604 -8.147771) (width 0.254) (layer F.Cu) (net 8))
 (segment (start 5.668269 -4.5) (end 2.25 -4.5) (width 0.254) (layer F.Cu) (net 8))
 (segment (start 9.31604 -8.147771) (end 5.668269 -4.5) (width 0.254) (layer F.Cu) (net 8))
 (segment (start 35.5 -9) (end 35.5 -11.5) (width 0.254) (layer F.Cu) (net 10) (status 30))
 (segment (start 35.5 -12.454) (end 34.29598 -13.65802) (width 0.254) (layer F.Cu) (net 10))
 (segment (start 35.5 -11.5) (end 35.5 -12.454) (width 0.254) (layer F.Cu) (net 10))
 (segment (start 10.607448 -13.65802) (end 8.75 -11.800572) (width 0.254) (layer F.Cu) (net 10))
 (segment (start 34.29598 -13.65802) (end 10.607448 -13.65802) (width 0.254) (layer F.Cu) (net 10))
 (segment (start 8.75 -11.800572) (end 8.75 -8.223797) (width 0.254) (layer F.Cu) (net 10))
 (segment (start 5.826203 -5.3) (end 2.25 -5.3) (width 0.254) (layer F.Cu) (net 10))
 (segment (start 8.75 -8.223797) (end 5.826203 -5.3) (width 0.254) (layer F.Cu) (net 10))
 (segment (start 36.75 -9) (end 36.75 -11.5) (width 0.254) (layer F.Cu) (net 12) (status 30))
 (segment (start 5.984137 -6.1) (end 2.25 -6.1) (width 0.254) (layer F.Cu) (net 12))
 (segment (start 8.29599 -8.411853) (end 5.984137 -6.1) (width 0.254) (layer F.Cu) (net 12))
 (segment (start 8.29599 -11.988629) (end 8.29599 -8.411853) (width 0.254) (layer F.Cu) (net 12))
 (segment (start 10.419391 -14.11203) (end 8.29599 -11.988629) (width 0.254) (layer F.Cu) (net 12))
 (segment (start 35.09197 -14.11203) (end 10.419391 -14.11203) (width 0.254) (layer F.Cu) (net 12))
 (segment (start 36.75 -12.454) (end 35.09197 -14.11203) (width 0.254) (layer F.Cu) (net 12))
 (segment (start 36.75 -11.5) (end 36.75 -12.454) (width 0.254) (layer F.Cu) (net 12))
 (segment (start 38 -9) (end 38 -11.5) (width 0.254) (layer F.Cu) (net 14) (status 30))
 (segment (start 38 -12.454) (end 35.704 -14.75) (width 0.254) (layer F.Cu) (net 14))
 (segment (start 38 -11.5) (end 38 -12.454) (width 0.254) (layer F.Cu) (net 14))
 (segment (start 10.415295 -14.75) (end 7.84198 -12.176686) (width 0.254) (layer F.Cu) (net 14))
 (segment (start 35.704 -14.75) (end 10.415295 -14.75) (width 0.254) (layer F.Cu) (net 14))
 (segment (start 7.84198 -12.176686) (end 7.84198 -8.599909) (width 0.254) (layer F.Cu) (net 14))
 (segment (start 6.142071 -6.9) (end 2.25 -6.9) (width 0.254) (layer F.Cu) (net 14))
 (segment (start 7.84198 -8.599909) (end 6.142071 -6.9) (width 0.254) (layer F.Cu) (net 14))
 (segment (start 39.25 -9) (end 39.25 -11.5) (width 0.254) (layer F.Cu) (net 16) (status 30))
 (segment (start 6.300005 -7.7) (end 2.25 -7.7) (width 0.254) (layer F.Cu) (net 16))
 (segment (start 7.29925 -8.699245) (end 6.300005 -7.7) (width 0.254) (layer F.Cu) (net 16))
 (segment (start 7.29925 -12.276023) (end 7.29925 -8.699245) (width 0.254) (layer F.Cu) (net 16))
 (segment (start 10.273227 -15.25) (end 7.29925 -12.276023) (width 0.254) (layer F.Cu) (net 16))
 (segment (start 39.25 -12.454) (end 36.454 -15.25) (width 0.254) (layer F.Cu) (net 16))
 (segment (start 36.454 -15.25) (end 10.273227 -15.25) (width 0.254) (layer F.Cu) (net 16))
 (segment (start 39.25 -11.5) (end 39.25 -12.454) (width 0.254) (layer F.Cu) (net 16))
 (segment (start 40.5 -9) (end 40.5 -11.5) (width 0.254) (layer F.Cu) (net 18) (status 30))
 (segment (start 40.5 -11.5) (end 40.5 -12.75) (width 0.254) (layer F.Cu) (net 18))
 (segment (start 6.08116 -11.7) (end 2.25 -11.7) (width 0.254) (layer F.Cu) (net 18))
 (segment (start 10.08517 -15.70401) (end 6.08116 -11.7) (width 0.254) (layer F.Cu) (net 18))
 (segment (start 37.24999 -15.70401) (end 10.08517 -15.70401) (width 0.254) (layer F.Cu) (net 18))
 (segment (start 40.5 -12.454) (end 37.24999 -15.70401) (width 0.254) (layer F.Cu) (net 18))
 (segment (start 40.5 -11.5) (end 40.5 -12.454) (width 0.254) (layer F.Cu) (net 18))
 (segment (start 41.75 -9) (end 41.75 -11.5) (width 0.254) (layer F.Cu) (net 20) (status 30))
 (segment (start 41.75 -12.454) (end 38.04598 -16.15802) (width 0.254) (layer F.Cu) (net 20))
 (segment (start 41.75 -11.5) (end 41.75 -12.454) (width 0.254) (layer F.Cu) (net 20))
 (segment (start 6.239093 -12.5) (end 2.25 -12.5) (width 0.254) (layer F.Cu) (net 20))
 (segment (start 9.897113 -16.15802) (end 6.239093 -12.5) (width 0.254) (layer F.Cu) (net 20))
 (segment (start 38.04598 -16.15802) (end 9.897113 -16.15802) (width 0.254) (layer F.Cu) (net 20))
 (segment (start 43 -9) (end 43 -11.5) (width 0.254) (layer F.Cu) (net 22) (status 30))
 (segment (start 43 -12.454) (end 38.84197 -16.61203) (width 0.254) (layer F.Cu) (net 22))
 (segment (start 43 -11.5) (end 43 -12.454) (width 0.254) (layer F.Cu) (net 22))
 (segment (start 6.397026 -13.3) (end 2.25 -13.3) (width 0.254) (layer F.Cu) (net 22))
 (segment (start 9.709056 -16.61203) (end 6.397026 -13.3) (width 0.254) (layer F.Cu) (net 22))
 (segment (start 38.84197 -16.61203) (end 9.709056 -16.61203) (width 0.254) (layer F.Cu) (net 22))
 (segment (start 44.25 -9) (end 44.25 -11.5) (width 0.254) (layer F.Cu) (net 24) (status 30))
 (segment (start 44.25 -12.454) (end 39.63796 -17.06604) (width 0.254) (layer F.Cu) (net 24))
 (segment (start 44.25 -11.5) (end 44.25 -12.454) (width 0.254) (layer F.Cu) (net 24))
 (segment (start 6.554959 -14.1) (end 2.25 -14.1) (width 0.254) (layer F.Cu) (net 24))
 (segment (start 9.520999 -17.06604) (end 6.554959 -14.1) (width 0.254) (layer F.Cu) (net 24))
 (segment (start 39.63796 -17.06604) (end 9.520999 -17.06604) (width 0.254) (layer F.Cu) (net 24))
 (segment (start 2.25 -5.3) (end 5.384132 -5.3) (width 0.254) (layer B.Cu) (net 11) (status 10))
 (via (at 10.8 -1.500003) (size 0.6) (drill 0.4) (layers F.Cu B.Cu) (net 11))
 (segment (start 9.184129 -1.500003) (end 10.8 -1.500003) (width 0.254) (layer B.Cu) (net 11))
 (segment (start 5.384132 -5.3) (end 9.184129 -1.500003) (width 0.254) (layer B.Cu) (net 11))
 (segment (start 17.5 -9) (end 17.5 -11.5) (width 0.254) (layer F.Cu) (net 11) (status 30))
 (via (at 17.5 -1.5) (size 0.6) (drill 0.4) (layers F.Cu B.Cu) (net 11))
 (segment (start 17.499997 -1.500003) (end 17.5 -1.5) (width 0.254) (layer B.Cu) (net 11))
 (segment (start 10.8 -1.500003) (end 17.499997 -1.500003) (width 0.254) (layer B.Cu) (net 11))
 (segment (start 17.5 -1.5) (end 17.5 -9) (width 0.254) (layer F.Cu) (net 11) (status 20))
 (segment (start 2.25 -15.7) (end 6.870826 -15.7) (width 0.254) (layer F.Cu) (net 3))
 (segment (start 43.55 -19.25) (end 10.420827 -19.25) (width 0.254) (layer F.Cu) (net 3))
 (segment (start 8.960414 -17.789587) (end 8.960413 -17.789587) (width 0.254) (layer F.Cu) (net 3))
 (segment (start 10.420827 -19.25) (end 8.960414 -17.789587) (width 0.254) (layer F.Cu) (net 3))
 (segment (start 6.870826 -15.7) (end 8.960413 -17.789587) (width 0.254) (layer F.Cu) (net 3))
 (segment (start 46.45 -18.25) (end 46.45 -18.75) (width 0.254) (layer F.Cu) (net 4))
 (segment (start 46.45 -18.75) (end 46.45 -19.25) (width 0.254) (layer F.Cu) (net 4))
 (segment (start 45.95 -20.05) (end 10.542839 -20.05) (width 0.3048) (layer F.Cu) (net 4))
 (segment (start 46.45 -19.25) (end 46.45 -19.55) (width 0.3048) (layer F.Cu) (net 4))
 (segment (start 46.45 -19.55) (end 45.95 -20.05) (width 0.3048) (layer F.Cu) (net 4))
 (segment (start 10.542839 -20.05) (end 6.992839 -16.5) (width 0.3048) (layer F.Cu) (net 4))
 (segment (start 6.992839 -16.5) (end 2.25 -16.5) (width 0.3048) (layer F.Cu) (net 4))
 (segment (start 6.712893 -14.9) (end 9.332942 -17.52005) (width 0.254) (layer F.Cu) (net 2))
 (segment (start 2.25 -14.9) (end 6.712893 -14.9) (width 0.254) (layer F.Cu) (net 2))
 (segment (start 10.562892 -18.75) (end 9.332942 -17.52005) (width 0.254) (layer F.Cu) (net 2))
 (segment (start 43.55 -18.75) (end 10.562892 -18.75) (width 0.254) (layer F.Cu) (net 2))
 (via (at 42.25 -17.75) (size 0.6) (drill 0.4) (layers F.Cu B.Cu) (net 1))
 (segment (start 41 -16.5) (end 42.25 -17.75) (width 0.3048) (layer B.Cu) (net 1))
 (segment (start 2.25 -16.5) (end 41 -16.5) (width 0.3048) (layer B.Cu) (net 1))
 (segment (start 43.55 -17.75) (end 42.25 -17.75) (width 0.254) (layer F.Cu) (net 1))
 (segment (start 2.25 -15.7) (end 43.45 -15.7) (width 0.254) (layer B.Cu) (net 26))
 (via (at 49 -19.25) (size 0.6) (drill 0.4) (layers F.Cu B.Cu) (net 26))
 (segment (start 45.45 -15.7) (end 49 -19.25) (width 0.254) (layer B.Cu) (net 26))
 (segment (start 43.45 -15.7) (end 45.45 -15.7) (width 0.254) (layer B.Cu) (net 26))
 (segment (start 49 -19.25) (end 48 -19.25) (width 0.254) (layer F.Cu) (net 26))
 (segment (start 48 -17.75) (end 46.45 -17.75) (width 0.254) (layer F.Cu) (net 5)))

